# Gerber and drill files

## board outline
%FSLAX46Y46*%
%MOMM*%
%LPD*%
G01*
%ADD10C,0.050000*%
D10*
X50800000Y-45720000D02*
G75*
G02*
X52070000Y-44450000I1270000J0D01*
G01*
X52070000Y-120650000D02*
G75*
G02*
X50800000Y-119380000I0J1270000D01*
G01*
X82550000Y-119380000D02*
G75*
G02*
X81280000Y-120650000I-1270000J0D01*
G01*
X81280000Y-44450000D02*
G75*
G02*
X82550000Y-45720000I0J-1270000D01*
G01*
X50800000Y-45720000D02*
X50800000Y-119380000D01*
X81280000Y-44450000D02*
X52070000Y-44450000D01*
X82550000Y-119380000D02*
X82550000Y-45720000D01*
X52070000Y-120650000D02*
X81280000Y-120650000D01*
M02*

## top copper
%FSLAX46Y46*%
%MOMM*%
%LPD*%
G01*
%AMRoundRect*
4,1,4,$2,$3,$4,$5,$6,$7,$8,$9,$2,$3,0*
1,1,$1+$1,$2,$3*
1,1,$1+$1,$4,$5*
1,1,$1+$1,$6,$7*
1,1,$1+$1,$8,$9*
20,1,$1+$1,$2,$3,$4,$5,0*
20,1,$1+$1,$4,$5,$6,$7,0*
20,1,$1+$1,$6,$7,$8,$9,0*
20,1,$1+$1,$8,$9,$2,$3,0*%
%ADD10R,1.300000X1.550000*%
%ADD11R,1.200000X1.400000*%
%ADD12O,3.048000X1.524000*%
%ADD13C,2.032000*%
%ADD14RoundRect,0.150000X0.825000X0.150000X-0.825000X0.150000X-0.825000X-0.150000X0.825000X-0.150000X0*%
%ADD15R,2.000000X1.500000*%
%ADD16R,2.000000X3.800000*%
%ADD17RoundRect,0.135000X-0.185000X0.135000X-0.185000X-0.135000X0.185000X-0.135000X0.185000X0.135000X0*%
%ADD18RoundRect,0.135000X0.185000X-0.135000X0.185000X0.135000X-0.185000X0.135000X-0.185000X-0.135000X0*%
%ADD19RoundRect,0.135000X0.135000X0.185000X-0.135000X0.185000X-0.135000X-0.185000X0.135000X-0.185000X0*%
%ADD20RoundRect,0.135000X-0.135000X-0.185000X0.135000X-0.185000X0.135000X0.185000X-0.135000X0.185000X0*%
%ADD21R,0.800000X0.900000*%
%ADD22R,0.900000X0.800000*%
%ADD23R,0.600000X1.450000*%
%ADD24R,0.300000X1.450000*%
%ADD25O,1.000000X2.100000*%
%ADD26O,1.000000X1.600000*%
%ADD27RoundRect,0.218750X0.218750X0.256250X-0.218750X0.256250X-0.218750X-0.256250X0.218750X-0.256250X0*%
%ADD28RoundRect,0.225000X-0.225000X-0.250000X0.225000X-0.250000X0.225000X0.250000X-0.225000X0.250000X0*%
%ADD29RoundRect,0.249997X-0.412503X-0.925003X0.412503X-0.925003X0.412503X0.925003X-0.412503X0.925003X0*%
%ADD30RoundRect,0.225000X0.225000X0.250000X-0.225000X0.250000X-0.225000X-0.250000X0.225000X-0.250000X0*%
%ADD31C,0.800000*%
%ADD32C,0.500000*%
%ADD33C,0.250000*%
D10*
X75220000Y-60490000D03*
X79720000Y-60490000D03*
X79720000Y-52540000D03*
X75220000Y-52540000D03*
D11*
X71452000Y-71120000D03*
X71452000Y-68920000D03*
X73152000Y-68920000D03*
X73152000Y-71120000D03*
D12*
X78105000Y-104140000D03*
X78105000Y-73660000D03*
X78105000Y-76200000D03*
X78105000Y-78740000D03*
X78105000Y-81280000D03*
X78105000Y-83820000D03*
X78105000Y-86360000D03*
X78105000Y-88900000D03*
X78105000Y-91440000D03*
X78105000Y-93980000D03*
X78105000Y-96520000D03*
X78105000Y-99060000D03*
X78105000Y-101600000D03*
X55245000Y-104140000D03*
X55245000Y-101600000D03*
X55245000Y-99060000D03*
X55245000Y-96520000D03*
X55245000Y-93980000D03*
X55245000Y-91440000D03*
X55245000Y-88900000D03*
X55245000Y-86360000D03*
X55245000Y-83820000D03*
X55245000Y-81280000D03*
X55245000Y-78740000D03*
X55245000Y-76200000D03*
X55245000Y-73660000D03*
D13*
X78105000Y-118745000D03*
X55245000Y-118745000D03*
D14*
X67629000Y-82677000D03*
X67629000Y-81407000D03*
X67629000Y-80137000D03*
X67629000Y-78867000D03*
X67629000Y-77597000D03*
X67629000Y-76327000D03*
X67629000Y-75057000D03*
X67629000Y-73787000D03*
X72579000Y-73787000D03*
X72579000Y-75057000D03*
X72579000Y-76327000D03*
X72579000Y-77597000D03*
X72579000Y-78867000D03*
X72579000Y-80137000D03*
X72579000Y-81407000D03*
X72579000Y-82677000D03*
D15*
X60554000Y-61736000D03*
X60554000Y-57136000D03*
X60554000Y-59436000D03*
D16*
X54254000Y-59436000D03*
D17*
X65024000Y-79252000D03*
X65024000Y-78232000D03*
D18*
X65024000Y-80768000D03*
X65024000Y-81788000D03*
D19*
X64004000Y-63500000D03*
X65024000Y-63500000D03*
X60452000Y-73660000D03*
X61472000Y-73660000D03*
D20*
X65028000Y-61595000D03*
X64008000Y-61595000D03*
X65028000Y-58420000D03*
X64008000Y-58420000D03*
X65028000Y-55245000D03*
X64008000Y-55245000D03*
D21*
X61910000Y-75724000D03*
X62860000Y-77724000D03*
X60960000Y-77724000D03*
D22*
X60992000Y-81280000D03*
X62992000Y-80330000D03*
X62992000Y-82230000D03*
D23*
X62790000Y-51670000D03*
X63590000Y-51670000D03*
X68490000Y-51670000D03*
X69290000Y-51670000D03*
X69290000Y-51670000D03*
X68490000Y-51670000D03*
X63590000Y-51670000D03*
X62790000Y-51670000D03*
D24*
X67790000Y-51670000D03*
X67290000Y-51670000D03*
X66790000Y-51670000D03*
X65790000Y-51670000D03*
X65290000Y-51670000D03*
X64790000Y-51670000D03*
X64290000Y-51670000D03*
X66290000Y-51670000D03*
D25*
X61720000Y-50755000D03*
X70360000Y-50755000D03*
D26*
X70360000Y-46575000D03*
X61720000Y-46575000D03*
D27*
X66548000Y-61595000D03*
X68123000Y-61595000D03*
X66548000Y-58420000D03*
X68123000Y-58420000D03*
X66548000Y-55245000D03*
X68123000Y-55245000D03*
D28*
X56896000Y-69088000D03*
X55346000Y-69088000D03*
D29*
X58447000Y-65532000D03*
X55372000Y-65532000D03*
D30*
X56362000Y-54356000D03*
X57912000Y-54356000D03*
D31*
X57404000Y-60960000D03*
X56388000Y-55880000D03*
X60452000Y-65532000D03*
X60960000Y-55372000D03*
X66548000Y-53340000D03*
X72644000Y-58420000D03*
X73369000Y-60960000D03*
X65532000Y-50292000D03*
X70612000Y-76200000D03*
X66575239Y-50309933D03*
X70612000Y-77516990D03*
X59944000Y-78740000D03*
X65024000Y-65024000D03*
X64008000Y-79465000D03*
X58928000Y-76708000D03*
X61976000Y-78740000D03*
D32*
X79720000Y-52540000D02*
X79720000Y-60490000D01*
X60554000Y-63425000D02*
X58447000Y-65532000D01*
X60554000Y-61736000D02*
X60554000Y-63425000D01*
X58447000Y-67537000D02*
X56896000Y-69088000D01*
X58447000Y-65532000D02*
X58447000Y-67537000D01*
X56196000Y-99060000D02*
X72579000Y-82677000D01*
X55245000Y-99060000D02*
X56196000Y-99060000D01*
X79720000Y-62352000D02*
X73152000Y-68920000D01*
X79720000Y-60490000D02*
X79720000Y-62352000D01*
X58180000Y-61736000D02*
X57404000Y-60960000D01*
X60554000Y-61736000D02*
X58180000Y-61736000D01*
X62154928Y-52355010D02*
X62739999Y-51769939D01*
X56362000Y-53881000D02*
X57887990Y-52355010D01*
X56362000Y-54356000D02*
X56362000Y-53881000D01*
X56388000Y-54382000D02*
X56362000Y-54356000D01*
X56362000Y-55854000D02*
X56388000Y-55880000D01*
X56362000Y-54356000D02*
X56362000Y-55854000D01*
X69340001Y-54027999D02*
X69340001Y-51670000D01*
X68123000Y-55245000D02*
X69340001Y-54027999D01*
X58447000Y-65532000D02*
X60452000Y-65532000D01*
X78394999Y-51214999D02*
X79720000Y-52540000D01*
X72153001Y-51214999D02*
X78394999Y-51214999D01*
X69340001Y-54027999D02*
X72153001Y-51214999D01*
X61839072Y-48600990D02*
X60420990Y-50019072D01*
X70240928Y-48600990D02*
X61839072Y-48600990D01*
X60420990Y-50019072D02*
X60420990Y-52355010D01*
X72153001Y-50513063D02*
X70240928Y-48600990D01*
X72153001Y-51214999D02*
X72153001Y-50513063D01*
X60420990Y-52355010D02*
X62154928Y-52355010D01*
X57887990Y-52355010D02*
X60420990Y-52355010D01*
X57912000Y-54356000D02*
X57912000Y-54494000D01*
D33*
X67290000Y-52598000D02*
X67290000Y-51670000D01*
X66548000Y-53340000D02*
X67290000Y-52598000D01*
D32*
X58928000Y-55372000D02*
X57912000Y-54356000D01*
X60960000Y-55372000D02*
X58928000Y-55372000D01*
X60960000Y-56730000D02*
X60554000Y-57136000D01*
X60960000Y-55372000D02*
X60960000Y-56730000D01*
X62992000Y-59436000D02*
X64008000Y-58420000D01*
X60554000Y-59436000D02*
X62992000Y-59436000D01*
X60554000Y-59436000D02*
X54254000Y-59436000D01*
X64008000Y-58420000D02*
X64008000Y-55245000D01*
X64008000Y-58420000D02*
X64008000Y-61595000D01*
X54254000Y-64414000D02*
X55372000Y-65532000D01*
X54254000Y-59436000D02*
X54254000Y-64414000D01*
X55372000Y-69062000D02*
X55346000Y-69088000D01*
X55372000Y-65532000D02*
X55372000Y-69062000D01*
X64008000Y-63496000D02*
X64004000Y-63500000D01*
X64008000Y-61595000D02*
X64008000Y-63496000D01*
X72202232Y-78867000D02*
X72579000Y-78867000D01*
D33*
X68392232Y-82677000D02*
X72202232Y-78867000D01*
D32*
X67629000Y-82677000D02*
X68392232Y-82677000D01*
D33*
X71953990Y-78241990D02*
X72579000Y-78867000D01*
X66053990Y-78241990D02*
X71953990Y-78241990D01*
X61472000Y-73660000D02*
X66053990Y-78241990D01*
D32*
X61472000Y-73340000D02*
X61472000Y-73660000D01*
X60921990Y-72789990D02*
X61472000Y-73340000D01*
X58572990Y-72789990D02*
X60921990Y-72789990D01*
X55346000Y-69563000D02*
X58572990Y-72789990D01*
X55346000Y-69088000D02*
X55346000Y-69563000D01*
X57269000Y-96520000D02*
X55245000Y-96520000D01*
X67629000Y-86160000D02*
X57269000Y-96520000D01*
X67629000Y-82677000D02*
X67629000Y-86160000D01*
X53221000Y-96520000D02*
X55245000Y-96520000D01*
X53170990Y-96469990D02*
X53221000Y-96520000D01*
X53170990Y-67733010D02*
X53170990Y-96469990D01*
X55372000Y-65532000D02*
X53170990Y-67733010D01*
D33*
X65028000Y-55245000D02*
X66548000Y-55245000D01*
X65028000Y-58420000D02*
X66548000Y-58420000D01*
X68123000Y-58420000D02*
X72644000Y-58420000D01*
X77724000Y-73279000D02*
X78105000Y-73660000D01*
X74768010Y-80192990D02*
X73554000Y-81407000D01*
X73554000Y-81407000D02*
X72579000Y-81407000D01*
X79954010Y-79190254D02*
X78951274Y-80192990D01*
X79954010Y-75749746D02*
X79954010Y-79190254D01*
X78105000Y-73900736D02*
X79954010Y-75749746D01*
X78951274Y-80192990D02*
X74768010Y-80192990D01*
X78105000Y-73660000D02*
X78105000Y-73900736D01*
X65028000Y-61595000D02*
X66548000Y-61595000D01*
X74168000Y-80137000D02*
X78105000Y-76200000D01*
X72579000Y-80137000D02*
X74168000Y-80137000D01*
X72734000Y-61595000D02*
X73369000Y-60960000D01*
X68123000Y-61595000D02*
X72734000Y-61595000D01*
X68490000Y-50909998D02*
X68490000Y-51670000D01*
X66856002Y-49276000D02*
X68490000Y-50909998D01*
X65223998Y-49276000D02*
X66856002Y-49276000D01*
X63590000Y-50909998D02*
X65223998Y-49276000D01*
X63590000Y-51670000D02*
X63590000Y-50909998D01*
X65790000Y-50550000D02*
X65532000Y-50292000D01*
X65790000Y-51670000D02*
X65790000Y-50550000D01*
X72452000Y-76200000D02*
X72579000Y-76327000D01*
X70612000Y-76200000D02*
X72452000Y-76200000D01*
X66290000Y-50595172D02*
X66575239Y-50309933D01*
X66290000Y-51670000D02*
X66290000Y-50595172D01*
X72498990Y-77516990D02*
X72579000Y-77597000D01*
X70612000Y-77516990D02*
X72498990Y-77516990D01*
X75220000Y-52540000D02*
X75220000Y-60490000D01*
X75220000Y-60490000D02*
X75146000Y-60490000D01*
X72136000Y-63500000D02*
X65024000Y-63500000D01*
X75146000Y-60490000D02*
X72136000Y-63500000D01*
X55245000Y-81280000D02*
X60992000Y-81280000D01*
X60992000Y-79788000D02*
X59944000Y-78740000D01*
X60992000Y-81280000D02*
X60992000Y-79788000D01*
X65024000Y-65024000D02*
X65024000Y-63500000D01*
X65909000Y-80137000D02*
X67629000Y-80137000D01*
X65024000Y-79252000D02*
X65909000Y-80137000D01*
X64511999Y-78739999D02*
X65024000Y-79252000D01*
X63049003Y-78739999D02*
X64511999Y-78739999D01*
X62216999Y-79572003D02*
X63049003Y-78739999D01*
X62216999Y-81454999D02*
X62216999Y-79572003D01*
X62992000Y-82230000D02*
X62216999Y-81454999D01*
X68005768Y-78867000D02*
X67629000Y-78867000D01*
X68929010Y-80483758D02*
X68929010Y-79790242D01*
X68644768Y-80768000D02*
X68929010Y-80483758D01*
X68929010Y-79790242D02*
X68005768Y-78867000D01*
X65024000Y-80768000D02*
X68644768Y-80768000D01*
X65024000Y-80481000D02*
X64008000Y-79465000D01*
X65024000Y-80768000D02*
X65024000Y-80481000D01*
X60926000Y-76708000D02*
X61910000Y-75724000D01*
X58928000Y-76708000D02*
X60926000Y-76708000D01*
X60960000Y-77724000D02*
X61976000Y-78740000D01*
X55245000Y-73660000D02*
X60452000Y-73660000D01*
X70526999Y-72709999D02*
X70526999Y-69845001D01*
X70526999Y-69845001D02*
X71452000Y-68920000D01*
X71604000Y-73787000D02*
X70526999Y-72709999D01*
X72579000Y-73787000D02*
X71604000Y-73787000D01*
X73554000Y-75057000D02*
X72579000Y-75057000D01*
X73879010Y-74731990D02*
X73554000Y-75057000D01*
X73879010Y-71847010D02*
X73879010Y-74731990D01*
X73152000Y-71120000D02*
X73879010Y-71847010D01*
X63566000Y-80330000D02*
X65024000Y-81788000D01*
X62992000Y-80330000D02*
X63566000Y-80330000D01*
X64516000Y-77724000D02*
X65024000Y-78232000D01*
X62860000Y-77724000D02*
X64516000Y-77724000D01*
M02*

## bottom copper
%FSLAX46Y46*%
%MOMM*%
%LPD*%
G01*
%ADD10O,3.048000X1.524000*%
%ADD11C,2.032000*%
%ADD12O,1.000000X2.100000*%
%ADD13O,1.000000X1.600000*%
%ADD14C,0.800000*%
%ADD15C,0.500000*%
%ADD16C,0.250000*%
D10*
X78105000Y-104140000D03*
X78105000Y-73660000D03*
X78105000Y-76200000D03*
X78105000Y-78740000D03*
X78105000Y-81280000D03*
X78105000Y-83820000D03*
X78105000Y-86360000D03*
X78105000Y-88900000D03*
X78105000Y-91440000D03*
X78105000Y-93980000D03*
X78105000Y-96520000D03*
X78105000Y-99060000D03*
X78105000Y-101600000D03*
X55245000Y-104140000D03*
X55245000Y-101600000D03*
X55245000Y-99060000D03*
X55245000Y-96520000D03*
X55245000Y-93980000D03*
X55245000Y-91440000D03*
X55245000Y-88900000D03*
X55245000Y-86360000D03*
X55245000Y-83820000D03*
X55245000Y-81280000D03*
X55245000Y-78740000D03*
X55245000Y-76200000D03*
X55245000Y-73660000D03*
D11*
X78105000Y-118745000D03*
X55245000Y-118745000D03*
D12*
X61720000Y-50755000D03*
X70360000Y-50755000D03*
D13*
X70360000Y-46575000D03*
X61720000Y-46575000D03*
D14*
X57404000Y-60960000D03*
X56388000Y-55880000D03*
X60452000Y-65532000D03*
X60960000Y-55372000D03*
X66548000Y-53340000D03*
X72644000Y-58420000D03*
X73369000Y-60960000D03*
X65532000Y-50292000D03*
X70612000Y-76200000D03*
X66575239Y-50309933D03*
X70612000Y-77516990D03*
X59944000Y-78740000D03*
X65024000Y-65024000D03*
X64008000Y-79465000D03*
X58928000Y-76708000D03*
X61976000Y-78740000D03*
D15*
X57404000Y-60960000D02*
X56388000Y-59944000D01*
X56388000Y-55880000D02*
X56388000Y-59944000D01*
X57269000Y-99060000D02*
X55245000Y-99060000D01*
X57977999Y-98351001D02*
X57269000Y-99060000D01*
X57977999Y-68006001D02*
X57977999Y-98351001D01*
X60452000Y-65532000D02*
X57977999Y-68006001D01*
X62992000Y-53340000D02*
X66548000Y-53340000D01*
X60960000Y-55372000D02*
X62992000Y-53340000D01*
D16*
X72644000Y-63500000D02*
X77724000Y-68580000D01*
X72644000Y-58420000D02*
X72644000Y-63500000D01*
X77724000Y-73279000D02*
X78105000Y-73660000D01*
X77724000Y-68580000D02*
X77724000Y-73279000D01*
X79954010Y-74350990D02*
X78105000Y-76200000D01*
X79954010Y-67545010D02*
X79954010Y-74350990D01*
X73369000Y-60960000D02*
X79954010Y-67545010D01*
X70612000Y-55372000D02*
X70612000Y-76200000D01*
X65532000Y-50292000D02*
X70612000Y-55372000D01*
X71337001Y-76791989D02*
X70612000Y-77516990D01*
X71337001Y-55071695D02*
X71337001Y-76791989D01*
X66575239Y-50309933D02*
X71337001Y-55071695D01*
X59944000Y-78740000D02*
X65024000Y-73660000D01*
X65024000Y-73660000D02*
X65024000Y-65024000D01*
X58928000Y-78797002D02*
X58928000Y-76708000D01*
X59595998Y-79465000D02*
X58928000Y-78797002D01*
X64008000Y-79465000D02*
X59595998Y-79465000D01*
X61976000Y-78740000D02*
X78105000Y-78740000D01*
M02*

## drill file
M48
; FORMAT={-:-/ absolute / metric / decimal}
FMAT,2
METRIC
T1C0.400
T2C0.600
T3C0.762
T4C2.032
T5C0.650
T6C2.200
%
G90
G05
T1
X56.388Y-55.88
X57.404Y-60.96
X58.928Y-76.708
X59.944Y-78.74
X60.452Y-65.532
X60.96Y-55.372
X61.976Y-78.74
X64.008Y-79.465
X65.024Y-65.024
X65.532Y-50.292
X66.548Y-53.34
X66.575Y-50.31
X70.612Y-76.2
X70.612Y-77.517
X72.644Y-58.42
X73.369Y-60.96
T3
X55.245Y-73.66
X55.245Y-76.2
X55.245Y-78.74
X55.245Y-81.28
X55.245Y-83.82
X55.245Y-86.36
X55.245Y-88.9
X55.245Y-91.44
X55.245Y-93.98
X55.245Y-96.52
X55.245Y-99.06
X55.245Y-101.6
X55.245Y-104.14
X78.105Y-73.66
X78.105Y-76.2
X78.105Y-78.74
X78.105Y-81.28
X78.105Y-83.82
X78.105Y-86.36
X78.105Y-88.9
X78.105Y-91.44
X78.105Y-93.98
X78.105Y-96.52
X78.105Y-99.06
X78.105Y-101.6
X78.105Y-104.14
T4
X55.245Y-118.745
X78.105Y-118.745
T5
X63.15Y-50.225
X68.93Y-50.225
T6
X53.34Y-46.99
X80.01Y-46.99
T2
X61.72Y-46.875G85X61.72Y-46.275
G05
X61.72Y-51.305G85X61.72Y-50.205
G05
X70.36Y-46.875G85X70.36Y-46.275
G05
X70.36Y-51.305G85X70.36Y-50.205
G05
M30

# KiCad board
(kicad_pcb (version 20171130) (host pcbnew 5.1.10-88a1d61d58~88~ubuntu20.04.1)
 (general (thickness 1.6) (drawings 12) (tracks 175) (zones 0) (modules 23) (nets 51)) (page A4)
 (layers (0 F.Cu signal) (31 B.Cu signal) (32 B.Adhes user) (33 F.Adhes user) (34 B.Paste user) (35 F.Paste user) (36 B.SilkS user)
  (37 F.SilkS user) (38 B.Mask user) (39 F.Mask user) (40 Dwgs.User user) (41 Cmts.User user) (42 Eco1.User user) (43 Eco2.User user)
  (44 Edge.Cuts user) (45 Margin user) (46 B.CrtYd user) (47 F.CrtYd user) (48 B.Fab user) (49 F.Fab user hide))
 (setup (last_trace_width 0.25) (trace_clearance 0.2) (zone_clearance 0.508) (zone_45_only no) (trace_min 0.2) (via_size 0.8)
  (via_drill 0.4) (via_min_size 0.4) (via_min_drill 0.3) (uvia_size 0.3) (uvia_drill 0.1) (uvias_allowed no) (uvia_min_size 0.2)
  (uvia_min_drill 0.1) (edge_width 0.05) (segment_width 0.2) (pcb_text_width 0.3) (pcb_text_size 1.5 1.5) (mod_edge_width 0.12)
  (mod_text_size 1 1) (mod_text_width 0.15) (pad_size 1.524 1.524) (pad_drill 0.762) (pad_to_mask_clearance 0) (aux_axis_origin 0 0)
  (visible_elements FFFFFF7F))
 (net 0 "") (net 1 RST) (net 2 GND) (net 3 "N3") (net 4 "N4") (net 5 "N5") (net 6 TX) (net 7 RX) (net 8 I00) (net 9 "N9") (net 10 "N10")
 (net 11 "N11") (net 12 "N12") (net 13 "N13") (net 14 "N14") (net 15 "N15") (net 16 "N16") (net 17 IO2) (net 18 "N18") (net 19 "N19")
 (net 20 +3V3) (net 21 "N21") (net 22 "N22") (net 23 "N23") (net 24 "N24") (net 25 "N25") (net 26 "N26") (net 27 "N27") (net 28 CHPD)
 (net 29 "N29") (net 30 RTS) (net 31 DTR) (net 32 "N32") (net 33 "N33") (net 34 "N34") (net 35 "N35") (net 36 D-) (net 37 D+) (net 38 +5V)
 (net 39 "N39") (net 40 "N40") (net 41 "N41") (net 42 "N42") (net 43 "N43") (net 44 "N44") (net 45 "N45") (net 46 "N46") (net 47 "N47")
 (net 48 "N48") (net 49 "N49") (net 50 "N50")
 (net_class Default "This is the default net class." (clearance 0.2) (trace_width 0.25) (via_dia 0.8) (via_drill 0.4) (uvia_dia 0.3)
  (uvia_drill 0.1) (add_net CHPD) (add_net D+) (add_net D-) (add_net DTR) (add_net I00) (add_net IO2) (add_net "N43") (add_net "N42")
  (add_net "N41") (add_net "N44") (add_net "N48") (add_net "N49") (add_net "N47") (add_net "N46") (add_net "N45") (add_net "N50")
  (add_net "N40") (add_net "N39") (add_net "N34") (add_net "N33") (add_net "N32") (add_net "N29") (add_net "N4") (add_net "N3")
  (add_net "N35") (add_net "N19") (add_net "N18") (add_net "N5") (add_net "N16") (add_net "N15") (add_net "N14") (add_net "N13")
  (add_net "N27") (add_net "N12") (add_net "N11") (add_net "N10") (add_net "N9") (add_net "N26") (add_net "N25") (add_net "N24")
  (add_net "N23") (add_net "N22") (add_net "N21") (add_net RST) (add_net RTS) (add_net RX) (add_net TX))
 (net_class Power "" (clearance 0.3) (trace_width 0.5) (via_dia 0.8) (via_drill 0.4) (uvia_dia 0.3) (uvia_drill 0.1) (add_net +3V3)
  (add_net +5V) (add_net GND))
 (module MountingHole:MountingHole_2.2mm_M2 (layer F.Cu) (at 53.34 46.99)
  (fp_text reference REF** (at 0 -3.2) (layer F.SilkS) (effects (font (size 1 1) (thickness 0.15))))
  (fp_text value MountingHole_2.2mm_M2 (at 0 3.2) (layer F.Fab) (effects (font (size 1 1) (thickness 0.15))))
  (pad 1 np_thru_hole circle (at 0 0) (size 2.2 2.2) (drill 2.2) (layers *.Cu *.Mask)))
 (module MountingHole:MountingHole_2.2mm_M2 (layer F.Cu) (at 80.01 46.99)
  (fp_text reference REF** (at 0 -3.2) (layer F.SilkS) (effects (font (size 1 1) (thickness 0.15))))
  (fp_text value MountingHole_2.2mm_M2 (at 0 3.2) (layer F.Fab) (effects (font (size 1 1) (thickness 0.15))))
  (pad 1 np_thru_hole circle (at 0 0) (size 2.2 2.2) (drill 2.2) (layers *.Cu *.Mask)))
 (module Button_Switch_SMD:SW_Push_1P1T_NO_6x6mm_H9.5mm (layer F.Cu) (at 77.47 56.515 270)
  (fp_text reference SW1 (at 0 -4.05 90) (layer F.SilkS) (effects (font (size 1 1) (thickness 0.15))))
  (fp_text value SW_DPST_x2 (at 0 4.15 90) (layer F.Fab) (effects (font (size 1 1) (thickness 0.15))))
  (pad 2 smd rect (at 3.975 2.25 270) (size 1.55 1.3) (layers F.Cu F.Paste F.Mask) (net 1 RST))
  (pad 1 smd rect (at 3.975 -2.25 270) (size 1.55 1.3) (layers F.Cu F.Paste F.Mask) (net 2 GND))
  (pad 1 smd rect (at -3.975 -2.25 270) (size 1.55 1.3) (layers F.Cu F.Paste F.Mask) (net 2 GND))
  (pad 2 smd rect (at -3.975 2.25 270) (size 1.55 1.3) (layers F.Cu F.Paste F.Mask) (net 1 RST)))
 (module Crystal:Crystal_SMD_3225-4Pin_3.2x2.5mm (layer F.Cu) (at 72.302 70.02 90)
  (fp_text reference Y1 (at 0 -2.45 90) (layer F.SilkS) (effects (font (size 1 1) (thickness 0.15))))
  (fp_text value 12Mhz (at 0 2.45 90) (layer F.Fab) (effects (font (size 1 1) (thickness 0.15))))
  (pad 4 smd rect (at -1.1 -0.85 90) (size 1.4 1.2) (layers F.Cu F.Paste F.Mask))
  (pad 3 smd rect (at 1.1 -0.85 90) (size 1.4 1.2) (layers F.Cu F.Paste F.Mask) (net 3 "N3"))
  (pad 2 smd rect (at 1.1 0.85 90) (size 1.4 1.2) (layers F.Cu F.Paste F.Mask) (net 2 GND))
  (pad 1 smd rect (at -1.1 0.85 90) (size 1.4 1.2) (layers F.Cu F.Paste F.Mask) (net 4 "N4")))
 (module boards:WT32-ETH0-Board (layer F.Cu) (at 66.675 92.71)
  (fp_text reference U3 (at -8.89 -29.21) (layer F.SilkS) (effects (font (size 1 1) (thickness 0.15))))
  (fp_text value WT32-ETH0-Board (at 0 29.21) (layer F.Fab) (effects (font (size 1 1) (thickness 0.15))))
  (pad 14 thru_hole oval (at 11.43 11.43) (size 3.048 1.524) (drill 0.762) (layers *.Cu *.Mask) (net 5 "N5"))
  (pad 26 thru_hole oval (at 11.43 -19.05) (size 3.048 1.524) (drill 0.762) (layers *.Cu *.Mask) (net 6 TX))
  (pad 25 thru_hole oval (at 11.43 -16.51) (size 3.048 1.524) (drill 0.762) (layers *.Cu *.Mask) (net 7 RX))
  (pad 24 thru_hole oval (at 11.43 -13.97) (size 3.048 1.524) (drill 0.762) (layers *.Cu *.Mask) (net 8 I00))
  (pad 23 thru_hole oval (at 11.43 -11.43) (size 3.048 1.524) (drill 0.762) (layers *.Cu *.Mask) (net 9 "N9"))
  (pad 22 thru_hole oval (at 11.43 -8.89) (size 3.048 1.524) (drill 0.762) (layers *.Cu *.Mask) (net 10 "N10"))
  (pad 21 thru_hole oval (at 11.43 -6.35) (size 3.048 1.524) (drill 0.762) (layers *.Cu *.Mask) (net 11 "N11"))
  (pad 20 thru_hole oval (at 11.43 -3.81) (size 3.048 1.524) (drill 0.762) (layers *.Cu *.Mask) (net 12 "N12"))
  (pad 19 thru_hole oval (at 11.43 -1.27) (size 3.048 1.524) (drill 0.762) (layers *.Cu *.Mask) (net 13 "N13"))
  (pad 18 thru_hole oval (at 11.43 1.27) (size 3.048 1.524) (drill 0.762) (layers *.Cu *.Mask) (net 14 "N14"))
  (pad 17 thru_hole oval (at 11.43 3.81) (size 3.048 1.524) (drill 0.762) (layers *.Cu *.Mask) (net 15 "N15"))
  (pad 16 thru_hole oval (at 11.43 6.35) (size 3.048 1.524) (drill 0.762) (layers *.Cu *.Mask) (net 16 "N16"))
  (pad 15 thru_hole oval (at 11.43 8.89) (size 3.048 1.524) (drill 0.762) (layers *.Cu *.Mask) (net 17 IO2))
  (pad 13 thru_hole oval (at -11.43 11.43) (size 3.048 1.524) (drill 0.762) (layers *.Cu *.Mask) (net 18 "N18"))
  (pad 12 thru_hole oval (at -11.43 8.89) (size 3.048 1.524) (drill 0.762) (layers *.Cu *.Mask) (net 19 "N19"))
  (pad 11 thru_hole oval (at -11.43 6.35) (size 3.048 1.524) (drill 0.762) (layers *.Cu *.Mask) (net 2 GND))
  (pad 10 thru_hole oval (at -11.43 3.81) (size 3.048 1.524) (drill 0.762) (layers *.Cu *.Mask) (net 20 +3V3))
  (pad 9 thru_hole oval (at -11.43 1.27) (size 3.048 1.524) (drill 0.762) (layers *.Cu *.Mask) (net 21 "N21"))
  (pad 8 thru_hole oval (at -11.43 -1.27) (size 3.048 1.524) (drill 0.762) (layers *.Cu *.Mask) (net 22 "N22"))
  (pad 7 thru_hole oval (at -11.43 -3.81) (size 3.048 1.524) (drill 0.762) (layers *.Cu *.Mask) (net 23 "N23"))
  (pad 6 thru_hole oval (at -11.43 -6.35) (size 3.048 1.524) (drill 0.762) (layers *.Cu *.Mask) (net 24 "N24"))
  (pad 5 thru_hole oval (at -11.43 -8.89) (size 3.048 1.524) (drill 0.762) (layers *.Cu *.Mask) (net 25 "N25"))
  (pad 4 thru_hole oval (at -11.43 -11.43) (size 3.048 1.524) (drill 0.762) (layers *.Cu *.Mask) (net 1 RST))
  (pad 3 thru_hole oval (at -11.43 -13.97) (size 3.048 1.524) (drill 0.762) (layers *.Cu *.Mask) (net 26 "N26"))
  (pad 2 thru_hole oval (at -11.43 -16.51) (size 3.048 1.524) (drill 0.762) (layers *.Cu *.Mask) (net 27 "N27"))
  (pad 1 thru_hole oval (at -11.43 -19.05) (size 3.048 1.524) (drill 0.762) (layers *.Cu *.Mask) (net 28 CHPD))
  (pad "" thru_hole circle (at 11.43 26.035) (size 2.032 2.032) (drill 2.032) (layers *.Mask F.Cu))
  (pad "" thru_hole circle (at -11.43 26.035) (size 2.032 2.032) (drill 2.032) (layers *.Mask F.Cu)))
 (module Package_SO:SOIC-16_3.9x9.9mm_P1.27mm (layer F.Cu) (at 70.104 78.232 180)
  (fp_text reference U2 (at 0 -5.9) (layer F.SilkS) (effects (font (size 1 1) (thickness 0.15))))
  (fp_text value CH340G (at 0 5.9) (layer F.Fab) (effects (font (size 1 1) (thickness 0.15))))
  (pad 16 smd roundrect (at 2.475 -4.445 180) (size 1.95 0.6) (layers F.Cu F.Paste F.Mask) (roundrect_rratio 0.25) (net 20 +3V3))
  (pad 15 smd roundrect (at 2.475 -3.175 180) (size 1.95 0.6) (layers F.Cu F.Paste F.Mask) (roundrect_rratio 0.25) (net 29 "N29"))
  (pad 14 smd roundrect (at 2.475 -1.905 180) (size 1.95 0.6) (layers F.Cu F.Paste F.Mask) (roundrect_rratio 0.25) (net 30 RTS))
  (pad 13 smd roundrect (at 2.475 -0.635 180) (size 1.95 0.6) (layers F.Cu F.Paste F.Mask) (roundrect_rratio 0.25) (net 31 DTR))
  (pad 12 smd roundrect (at 2.475 0.635 180) (size 1.95 0.6) (layers F.Cu F.Paste F.Mask) (roundrect_rratio 0.25) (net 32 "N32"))
  (pad 11 smd roundrect (at 2.475 1.905 180) (size 1.95 0.6) (layers F.Cu F.Paste F.Mask) (roundrect_rratio 0.25) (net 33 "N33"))
  (pad 10 smd roundrect (at 2.475 3.175 180) (size 1.95 0.6) (layers F.Cu F.Paste F.Mask) (roundrect_rratio 0.25) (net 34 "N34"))
  (pad 9 smd roundrect (at 2.475 4.445 180) (size 1.95 0.6) (layers F.Cu F.Paste F.Mask) (roundrect_rratio 0.25) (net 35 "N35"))
  (pad 8 smd roundrect (at -2.475 4.445 180) (size 1.95 0.6) (layers F.Cu F.Paste F.Mask) (roundrect_rratio 0.25) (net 3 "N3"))
  (pad 7 smd roundrect (at -2.475 3.175 180) (size 1.95 0.6) (layers F.Cu F.Paste F.Mask) (roundrect_rratio 0.25) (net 4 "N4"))
  (pad 6 smd roundrect (at -2.475 1.905 180) (size 1.95 0.6) (layers F.Cu F.Paste F.Mask) (roundrect_rratio 0.25) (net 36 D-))
  (pad 5 smd roundrect (at -2.475 0.635 180) (size 1.95 0.6) (layers F.Cu F.Paste F.Mask) (roundrect_rratio 0.25) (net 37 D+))
  (pad 4 smd roundrect (at -2.475 -0.635 180) (size 1.95 0.6) (layers F.Cu F.Paste F.Mask) (roundrect_rratio 0.25) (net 20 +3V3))
  (pad 3 smd roundrect (at -2.475 -1.905 180) (size 1.95 0.6) (layers F.Cu F.Paste F.Mask) (roundrect_rratio 0.25) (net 7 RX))
  (pad 2 smd roundrect (at -2.475 -3.175 180) (size 1.95 0.6) (layers F.Cu F.Paste F.Mask) (roundrect_rratio 0.25) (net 6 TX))
  (pad 1 smd roundrect (at -2.475 -4.445 180) (size 1.95 0.6) (layers F.Cu F.Paste F.Mask) (roundrect_rratio 0.25) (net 2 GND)))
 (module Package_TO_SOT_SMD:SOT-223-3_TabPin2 (layer F.Cu) (at 57.404 59.436 180)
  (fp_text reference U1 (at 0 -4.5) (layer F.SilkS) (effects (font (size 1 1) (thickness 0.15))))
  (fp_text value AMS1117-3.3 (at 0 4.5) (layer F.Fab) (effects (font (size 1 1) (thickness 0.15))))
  (pad 1 smd rect (at -3.15 -2.3 180) (size 2 1.5) (layers F.Cu F.Paste F.Mask) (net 2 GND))
  (pad 3 smd rect (at -3.15 2.3 180) (size 2 1.5) (layers F.Cu F.Paste F.Mask) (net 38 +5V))
  (pad 2 smd rect (at -3.15 0 180) (size 2 1.5) (layers F.Cu F.Paste F.Mask) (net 20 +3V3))
  (pad 2 smd rect (at 3.15 0 180) (size 2 3.8) (layers F.Cu F.Paste F.Mask) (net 20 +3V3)))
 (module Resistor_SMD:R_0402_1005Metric (layer F.Cu) (at 65.024 78.742 270)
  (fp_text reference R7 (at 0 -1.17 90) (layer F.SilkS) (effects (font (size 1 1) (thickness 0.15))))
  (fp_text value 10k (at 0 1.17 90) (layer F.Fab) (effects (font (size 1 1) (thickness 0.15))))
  (pad 2 smd roundrect (at 0.51 0 270) (size 0.54 0.64) (layers F.Cu F.Paste F.Mask) (roundrect_rratio 0.25) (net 30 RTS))
  (pad 1 smd roundrect (at -0.51 0 270) (size 0.54 0.64) (layers F.Cu F.Paste F.Mask) (roundrect_rratio 0.25) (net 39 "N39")))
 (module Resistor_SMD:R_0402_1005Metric (layer F.Cu) (at 65.024 81.278 90)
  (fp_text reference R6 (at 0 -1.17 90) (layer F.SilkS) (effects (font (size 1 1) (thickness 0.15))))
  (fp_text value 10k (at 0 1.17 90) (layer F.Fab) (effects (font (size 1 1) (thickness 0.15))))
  (pad 2 smd roundrect (at 0.51 0 90) (size 0.54 0.64) (layers F.Cu F.Paste F.Mask) (roundrect_rratio 0.25) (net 31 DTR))
  (pad 1 smd roundrect (at -0.51 0 90) (size 0.54 0.64) (layers F.Cu F.Paste F.Mask) (roundrect_rratio 0.25) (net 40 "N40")))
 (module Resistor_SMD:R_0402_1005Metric (layer F.Cu) (at 64.514 63.5 180)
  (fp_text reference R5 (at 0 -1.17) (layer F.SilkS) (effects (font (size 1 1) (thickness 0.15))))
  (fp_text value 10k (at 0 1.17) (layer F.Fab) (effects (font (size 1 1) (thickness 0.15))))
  (pad 2 smd roundrect (at 0.51 0 180) (size 0.54 0.64) (layers F.Cu F.Paste F.Mask) (roundrect_rratio 0.25) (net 20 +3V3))
  (pad 1 smd roundrect (at -0.51 0 180) (size 0.54 0.64) (layers F.Cu F.Paste F.Mask) (roundrect_rratio 0.25) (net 1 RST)))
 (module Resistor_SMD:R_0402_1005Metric (layer F.Cu) (at 60.962 73.66 180)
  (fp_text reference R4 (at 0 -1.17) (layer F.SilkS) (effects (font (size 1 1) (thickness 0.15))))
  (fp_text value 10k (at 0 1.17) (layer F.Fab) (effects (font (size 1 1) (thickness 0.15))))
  (pad 2 smd roundrect (at 0.51 0 180) (size 0.54 0.64) (layers F.Cu F.Paste F.Mask) (roundrect_rratio 0.25) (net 28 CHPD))
  (pad 1 smd roundrect (at -0.51 0 180) (size 0.54 0.64) (layers F.Cu F.Paste F.Mask) (roundrect_rratio 0.25) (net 20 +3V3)))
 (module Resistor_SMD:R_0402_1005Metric (layer F.Cu) (at 64.518 61.595)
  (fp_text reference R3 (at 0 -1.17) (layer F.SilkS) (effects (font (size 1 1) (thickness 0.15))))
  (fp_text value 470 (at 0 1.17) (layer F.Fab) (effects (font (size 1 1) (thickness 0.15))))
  (pad 2 smd roundrect (at 0.51 0) (size 0.54 0.64) (layers F.Cu F.Paste F.Mask) (roundrect_rratio 0.25) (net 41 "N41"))
  (pad 1 smd roundrect (at -0.51 0) (size 0.54 0.64) (layers F.Cu F.Paste F.Mask) (roundrect_rratio 0.25) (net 20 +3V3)))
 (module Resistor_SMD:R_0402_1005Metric (layer F.Cu) (at 64.518 58.42)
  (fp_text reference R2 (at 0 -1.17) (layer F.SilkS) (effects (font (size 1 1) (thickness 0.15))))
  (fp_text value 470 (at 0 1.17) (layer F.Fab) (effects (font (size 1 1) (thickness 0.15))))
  (pad 2 smd roundrect (at 0.51 0) (size 0.54 0.64) (layers F.Cu F.Paste F.Mask) (roundrect_rratio 0.25) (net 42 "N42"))
  (pad 1 smd roundrect (at -0.51 0) (size 0.54 0.64) (layers F.Cu F.Paste F.Mask) (roundrect_rratio 0.25) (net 20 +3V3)))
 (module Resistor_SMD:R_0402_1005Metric (layer F.Cu) (at 64.518 55.245)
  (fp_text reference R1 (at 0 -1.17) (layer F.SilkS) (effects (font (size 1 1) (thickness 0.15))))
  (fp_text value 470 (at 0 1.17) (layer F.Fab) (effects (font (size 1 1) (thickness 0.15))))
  (pad 2 smd roundrect (at 0.51 0) (size 0.54 0.64) (layers F.Cu F.Paste F.Mask) (roundrect_rratio 0.25) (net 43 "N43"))
  (pad 1 smd roundrect (at -0.51 0) (size 0.54 0.64) (layers F.Cu F.Paste F.Mask) (roundrect_rratio 0.25) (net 20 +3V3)))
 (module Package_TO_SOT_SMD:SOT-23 (layer F.Cu) (at 61.91 76.724 90)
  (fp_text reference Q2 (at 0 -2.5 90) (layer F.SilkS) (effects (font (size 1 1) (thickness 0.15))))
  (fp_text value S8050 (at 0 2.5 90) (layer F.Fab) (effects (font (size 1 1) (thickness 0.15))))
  (pad 3 smd rect (at 1 0 90) (size 0.9 0.8) (layers F.Cu F.Paste F.Mask) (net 31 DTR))
  (pad 2 smd rect (at -1 0.95 90) (size 0.9 0.8) (layers F.Cu F.Paste F.Mask) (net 39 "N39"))
  (pad 1 smd rect (at -1 -0.95 90) (size 0.9 0.8) (layers F.Cu F.Paste F.Mask) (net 8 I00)))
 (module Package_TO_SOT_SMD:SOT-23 (layer F.Cu) (at 61.992 81.28 180)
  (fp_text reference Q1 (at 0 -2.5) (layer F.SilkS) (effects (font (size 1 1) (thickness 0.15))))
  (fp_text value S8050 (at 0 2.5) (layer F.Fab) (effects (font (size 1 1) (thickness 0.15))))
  (pad 3 smd rect (at 1 0 180) (size 0.9 0.8) (layers F.Cu F.Paste F.Mask) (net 1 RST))
  (pad 2 smd rect (at -1 0.95 180) (size 0.9 0.8) (layers F.Cu F.Paste F.Mask) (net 40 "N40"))
  (pad 1 smd rect (at -1 -0.95 180) (size 0.9 0.8) (layers F.Cu F.Paste F.Mask) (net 30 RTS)))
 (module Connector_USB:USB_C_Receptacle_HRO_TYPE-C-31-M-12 (layer F.Cu) (at 66.04 47.625 180)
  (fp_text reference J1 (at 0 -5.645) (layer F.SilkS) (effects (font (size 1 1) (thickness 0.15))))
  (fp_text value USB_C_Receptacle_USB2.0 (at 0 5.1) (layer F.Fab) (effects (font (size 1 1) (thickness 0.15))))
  (pad B1 smd rect (at 3.25 -4.045 180) (size 0.6 1.45) (layers F.Cu F.Paste F.Mask) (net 2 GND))
  (pad A9 smd rect (at 2.45 -4.045 180) (size 0.6 1.45) (layers F.Cu F.Paste F.Mask) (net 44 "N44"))
  (pad B9 smd rect (at -2.45 -4.045 180) (size 0.6 1.45) (layers F.Cu F.Paste F.Mask) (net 44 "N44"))
  (pad B12 smd rect (at -3.25 -4.045 180) (size 0.6 1.45) (layers F.Cu F.Paste F.Mask) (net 2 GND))
  (pad A1 smd rect (at -3.25 -4.045 180) (size 0.6 1.45) (layers F.Cu F.Paste F.Mask) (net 2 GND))
  (pad A4 smd rect (at -2.45 -4.045 180) (size 0.6 1.45) (layers F.Cu F.Paste F.Mask) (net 44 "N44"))
  (pad B4 smd rect (at 2.45 -4.045 180) (size 0.6 1.45) (layers F.Cu F.Paste F.Mask) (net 44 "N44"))
  (pad A12 smd rect (at 3.25 -4.045 180) (size 0.6 1.45) (layers F.Cu F.Paste F.Mask) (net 2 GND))
  (pad B8 smd rect (at -1.75 -4.045 180) (size 0.3 1.45) (layers F.Cu F.Paste F.Mask) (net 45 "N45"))
  (pad A5 smd rect (at -1.25 -4.045 180) (size 0.3 1.45) (layers F.Cu F.Paste F.Mask) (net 38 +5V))
  (pad B7 smd rect (at -0.75 -4.045 180) (size 0.3 1.45) (layers F.Cu F.Paste F.Mask) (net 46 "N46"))
  (pad A7 smd rect (at 0.25 -4.045 180) (size 0.3 1.45) (layers F.Cu F.Paste F.Mask) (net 36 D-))
  (pad B6 smd rect (at 0.75 -4.045 180) (size 0.3 1.45) (layers F.Cu F.Paste F.Mask) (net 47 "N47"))
  (pad A8 smd rect (at 1.25 -4.045 180) (size 0.3 1.45) (layers F.Cu F.Paste F.Mask) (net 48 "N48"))
  (pad B5 smd rect (at 1.75 -4.045 180) (size 0.3 1.45) (layers F.Cu F.Paste F.Mask) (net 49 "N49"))
  (pad A6 smd rect (at -0.25 -4.045 180) (size 0.3 1.45) (layers F.Cu F.Paste F.Mask) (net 37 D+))
  (pad S1 thru_hole oval (at 4.32 -3.13 180) (size 1 2.1) (drill oval 0.6 1.7) (layers *.Cu *.Mask) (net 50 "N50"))
  (pad S1 thru_hole oval (at -4.32 -3.13 180) (size 1 2.1) (drill oval 0.6 1.7) (layers *.Cu *.Mask) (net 50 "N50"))
  (pad "" np_thru_hole circle (at -2.89 -2.6 180) (size 0.65 0.65) (drill 0.65) (layers *.Cu *.Mask))
  (pad S1 thru_hole oval (at -4.32 1.05 180) (size 1 1.6) (drill oval 0.6 1.2) (layers *.Cu *.Mask) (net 50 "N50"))
  (pad "" np_thru_hole circle (at 2.89 -2.6 180) (size 0.65 0.65) (drill 0.65) (layers *.Cu *.Mask))
  (pad S1 thru_hole oval (at 4.32 1.05 180) (size 1 1.6) (drill oval 0.6 1.2) (layers *.Cu *.Mask) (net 50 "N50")))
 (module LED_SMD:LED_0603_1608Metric (layer F.Cu) (at 67.3355 61.595 180)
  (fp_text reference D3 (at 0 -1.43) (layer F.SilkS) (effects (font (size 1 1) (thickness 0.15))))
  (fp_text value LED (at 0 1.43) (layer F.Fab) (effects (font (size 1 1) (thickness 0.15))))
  (pad 2 smd roundrect (at 0.7875 0 180) (size 0.875 0.95) (layers F.Cu F.Paste F.Mask) (roundrect_rratio 0.25) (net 41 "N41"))
  (pad 1 smd roundrect (at -0.7875 0 180) (size 0.875 0.95) (layers F.Cu F.Paste F.Mask) (roundrect_rratio 0.25) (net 7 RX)))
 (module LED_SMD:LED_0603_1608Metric (layer F.Cu) (at 67.3355 58.42 180)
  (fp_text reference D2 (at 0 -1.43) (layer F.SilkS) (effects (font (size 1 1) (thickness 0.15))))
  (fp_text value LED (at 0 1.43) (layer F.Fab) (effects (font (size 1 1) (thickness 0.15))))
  (pad 2 smd roundrect (at 0.7875 0 180) (size 0.875 0.95) (layers F.Cu F.Paste F.Mask) (roundrect_rratio 0.25) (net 42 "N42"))
  (pad 1 smd roundrect (at -0.7875 0 180) (size 0.875 0.95) (layers F.Cu F.Paste F.Mask) (roundrect_rratio 0.25) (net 6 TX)))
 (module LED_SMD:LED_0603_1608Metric (layer F.Cu) (at 67.3355 55.245 180)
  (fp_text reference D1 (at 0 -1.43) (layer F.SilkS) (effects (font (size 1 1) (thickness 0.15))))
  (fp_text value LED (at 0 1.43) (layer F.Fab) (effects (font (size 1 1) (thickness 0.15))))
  (pad 2 smd roundrect (at 0.7875 0 180) (size 0.875 0.95) (layers F.Cu F.Paste F.Mask) (roundrect_rratio 0.25) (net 43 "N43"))
  (pad 1 smd roundrect (at -0.7875 0 180) (size 0.875 0.95) (layers F.Cu F.Paste F.Mask) (roundrect_rratio 0.25) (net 2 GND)))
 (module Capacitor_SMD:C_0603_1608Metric (layer F.Cu) (at 56.121 69.088)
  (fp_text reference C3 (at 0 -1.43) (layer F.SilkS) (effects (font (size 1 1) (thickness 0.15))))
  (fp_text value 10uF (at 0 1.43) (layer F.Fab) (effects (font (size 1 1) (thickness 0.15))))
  (pad 2 smd roundrect (at 0.775 0) (size 0.9 0.95) (layers F.Cu F.Paste F.Mask) (roundrect_rratio 0.25) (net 2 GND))
  (pad 1 smd roundrect (at -0.775 0) (size 0.9 0.95) (layers F.Cu F.Paste F.Mask) (roundrect_rratio 0.25) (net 20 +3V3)))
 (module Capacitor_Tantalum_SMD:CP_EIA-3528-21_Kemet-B (layer F.Cu) (at 56.9095 65.532)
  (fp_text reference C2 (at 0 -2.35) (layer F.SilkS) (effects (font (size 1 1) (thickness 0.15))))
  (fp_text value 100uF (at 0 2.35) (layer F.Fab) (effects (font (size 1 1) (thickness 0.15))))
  (pad 2 smd roundrect (at 1.5375 0) (size 1.325 2.35) (layers F.Cu F.Paste F.Mask) (roundrect_rratio 0.1886769811320755) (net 2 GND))
  (pad 1 smd roundrect (at -1.5375 0) (size 1.325 2.35) (layers F.Cu F.Paste F.Mask) (roundrect_rratio 0.1886769811320755) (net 20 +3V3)))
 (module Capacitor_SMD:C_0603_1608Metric (layer F.Cu) (at 57.137 54.356 180)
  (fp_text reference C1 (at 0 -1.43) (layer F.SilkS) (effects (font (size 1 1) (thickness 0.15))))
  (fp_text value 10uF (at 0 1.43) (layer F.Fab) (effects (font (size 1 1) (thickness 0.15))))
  (pad 2 smd roundrect (at 0.775 0 180) (size 0.9 0.95) (layers F.Cu F.Paste F.Mask) (roundrect_rratio 0.25) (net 2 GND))
  (pad 1 smd roundrect (at -0.775 0 180) (size 0.9 0.95) (layers F.Cu F.Paste F.Mask) (roundrect_rratio 0.25) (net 38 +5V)))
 (gr_arc (start 52.07 45.72) (end 52.07 44.45) (angle -90) (layer Edge.Cuts) (width 0.05))
 (gr_arc (start 52.07 119.38) (end 50.8 119.38) (angle -90) (layer Edge.Cuts) (width 0.05))
 (gr_arc (start 81.28 119.38) (end 81.28 120.65) (angle -90) (layer Edge.Cuts) (width 0.05))
 (gr_arc (start 81.28 45.72) (end 82.55 45.72) (angle -90) (layer Edge.Cuts) (width 0.05))
 (gr_line (start 50.8 45.72) (end 50.8 119.38) (layer Edge.Cuts) (width 0.05))
 (gr_line (start 81.28 44.45) (end 52.07 44.45) (layer Edge.Cuts) (width 0.05))
 (gr_line (start 82.55 119.38) (end 82.55 45.72) (layer Edge.Cuts) (width 0.05))
 (gr_line (start 52.07 120.65) (end 81.28 120.65) (layer Edge.Cuts) (width 0.05))
 (segment (start 79.72 52.54) (end 79.72 60.49) (width 0.5) (layer F.Cu) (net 2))
 (segment (start 60.554 63.425) (end 58.447 65.532) (width 0.5) (layer F.Cu) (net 2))
 (segment (start 60.554 61.736) (end 60.554 63.425) (width 0.5) (layer F.Cu) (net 2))
 (segment (start 58.447 67.537) (end 56.896 69.088) (width 0.5) (layer F.Cu) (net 2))
 (segment (start 58.447 65.532) (end 58.447 67.537) (width 0.5) (layer F.Cu) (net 2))
 (segment (start 56.196 99.06) (end 72.579 82.677) (width 0.5) (layer F.Cu) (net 2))
 (segment (start 55.245 99.06) (end 56.196 99.06) (width 0.5) (layer F.Cu) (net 2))
 (segment (start 79.72 62.352) (end 73.152 68.92) (width 0.5) (layer F.Cu) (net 2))
 (segment (start 79.72 60.49) (end 79.72 62.352) (width 0.5) (layer F.Cu) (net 2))
 (via (at 57.404 60.96) (size 0.8) (drill 0.4) (layers F.Cu B.Cu) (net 2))
 (segment (start 58.18 61.736) (end 57.404 60.96) (width 0.5) (layer F.Cu) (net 2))
 (segment (start 60.554 61.736) (end 58.18 61.736) (width 0.5) (layer F.Cu) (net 2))
 (via (at 56.388 55.88) (size 0.8) (drill 0.4) (layers F.Cu B.Cu) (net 2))
 (segment (start 57.404 60.96) (end 56.388 59.944) (width 0.5) (layer B.Cu) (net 2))
 (segment (start 62.154928 52.35501) (end 62.739999 51.769939) (width 0.5) (layer F.Cu) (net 2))
 (segment (start 56.362 53.881) (end 57.88799 52.35501) (width 0.5) (layer F.Cu) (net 2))
 (segment (start 56.362 54.356) (end 56.362 53.881) (width 0.5) (layer F.Cu) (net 2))
 (segment (start 56.388 54.382) (end 56.362 54.356) (width 0.5) (layer F.Cu) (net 2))
 (segment (start 56.362 55.854) (end 56.388 55.88) (width 0.5) (layer F.Cu) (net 2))
 (segment (start 56.362 54.356) (end 56.362 55.854) (width 0.5) (layer F.Cu) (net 2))
 (segment (start 56.388 55.88) (end 56.388 59.944) (width 0.5) (layer B.Cu) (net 2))
 (segment (start 69.340001 54.027999) (end 69.340001 51.67) (width 0.5) (layer F.Cu) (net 2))
 (segment (start 68.123 55.245) (end 69.340001 54.027999) (width 0.5) (layer F.Cu) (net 2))
 (via (at 60.452 65.532) (size 0.8) (drill 0.4) (layers F.Cu B.Cu) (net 2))
 (segment (start 58.447 65.532) (end 60.452 65.532) (width 0.5) (layer F.Cu) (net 2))
 (segment (start 57.269 99.06) (end 55.245 99.06) (width 0.5) (layer B.Cu) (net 2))
 (segment (start 57.977999 98.351001) (end 57.269 99.06) (width 0.5) (layer B.Cu) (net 2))
 (segment (start 57.977999 68.006001) (end 57.977999 98.351001) (width 0.5) (layer B.Cu) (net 2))
 (segment (start 60.452 65.532) (end 57.977999 68.006001) (width 0.5) (layer B.Cu) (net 2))
 (segment (start 78.394999 51.214999) (end 79.72 52.54) (width 0.5) (layer F.Cu) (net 2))
 (segment (start 72.153001 51.214999) (end 78.394999 51.214999) (width 0.5) (layer F.Cu) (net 2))
 (segment (start 69.340001 54.027999) (end 72.153001 51.214999) (width 0.5) (layer F.Cu) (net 2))
 (segment (start 61.839072 48.60099) (end 60.42099 50.019072) (width 0.5) (layer F.Cu) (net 2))
 (segment (start 70.240928 48.60099) (end 61.839072 48.60099) (width 0.5) (layer F.Cu) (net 2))
 (segment (start 60.42099 50.019072) (end 60.42099 52.35501) (width 0.5) (layer F.Cu) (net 2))
 (segment (start 72.153001 50.513063) (end 70.240928 48.60099) (width 0.5) (layer F.Cu) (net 2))
 (segment (start 72.153001 51.214999) (end 72.153001 50.513063) (width 0.5) (layer F.Cu) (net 2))
 (segment (start 60.42099 52.35501) (end 62.154928 52.35501) (width 0.5) (layer F.Cu) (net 2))
 (segment (start 57.88799 52.35501) (end 60.42099 52.35501) (width 0.5) (layer F.Cu) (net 2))
 (segment (start 57.912 54.356) (end 57.912 54.494) (width 0.5) (layer F.Cu) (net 38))
 (via (at 60.96 55.372) (size 0.8) (drill 0.4) (layers F.Cu B.Cu) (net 38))
 (via (at 66.548 53.34) (size 0.8) (drill 0.4) (layers F.Cu B.Cu) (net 38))
 (segment (start 62.992 53.34) (end 66.548 53.34) (width 0.5) (layer B.Cu) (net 38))
 (segment (start 60.96 55.372) (end 62.992 53.34) (width 0.5) (layer B.Cu) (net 38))
 (segment (start 67.29 52.598) (end 67.29 51.67) (width 0.25) (layer F.Cu) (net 38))
 (segment (start 66.548 53.34) (end 67.29 52.598) (width 0.25) (layer F.Cu) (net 38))
 (segment (start 58.928 55.372) (end 57.912 54.356) (width 0.5) (layer F.Cu) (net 38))
 (segment (start 60.96 55.372) (end 58.928 55.372) (width 0.5) (layer F.Cu) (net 38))
 (segment (start 60.96 56.73) (end 60.554 57.136) (width 0.5) (layer F.Cu) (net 38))
 (segment (start 60.96 55.372) (end 60.96 56.73) (width 0.5) (layer F.Cu) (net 38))
 (segment (start 62.992 59.436) (end 64.008 58.42) (width 0.5) (layer F.Cu) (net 20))
 (segment (start 60.554 59.436) (end 62.992 59.436) (width 0.5) (layer F.Cu) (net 20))
 (segment (start 60.554 59.436) (end 54.254 59.436) (width 0.5) (layer F.Cu) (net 20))
 (segment (start 64.008 58.42) (end 64.008 55.245) (width 0.5) (layer F.Cu) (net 20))
 (segment (start 64.008 58.42) (end 64.008 61.595) (width 0.5) (layer F.Cu) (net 20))
 (segment (start 54.254 64.414) (end 55.372 65.532) (width 0.5) (layer F.Cu) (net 20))
 (segment (start 54.254 59.436) (end 54.254 64.414) (width 0.5) (layer F.Cu) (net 20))
 (segment (start 55.372 69.062) (end 55.346 69.088) (width 0.5) (layer F.Cu) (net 20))
 (segment (start 55.372 65.532) (end 55.372 69.062) (width 0.5) (layer F.Cu) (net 20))
 (segment (start 64.008 63.496) (end 64.004 63.5) (width 0.5) (layer F.Cu) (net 20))
 (segment (start 64.008 61.595) (end 64.008 63.496) (width 0.5) (layer F.Cu) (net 20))
 (segment (start 72.202232 78.867) (end 72.579 78.867) (width 0.5) (layer F.Cu) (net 20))
 (segment (start 68.392232 82.677) (end 72.202232 78.867) (width 0.25) (layer F.Cu) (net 20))
 (segment (start 67.629 82.677) (end 68.392232 82.677) (width 0.5) (layer F.Cu) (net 20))
 (segment (start 71.95399 78.24199) (end 72.579 78.867) (width 0.25) (layer F.Cu) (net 20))
 (segment (start 66.05399 78.24199) (end 71.95399 78.24199) (width 0.25) (layer F.Cu) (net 20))
 (segment (start 61.472 73.66) (end 66.05399 78.24199) (width 0.25) (layer F.Cu) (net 20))
 (segment (start 61.472 73.34) (end 61.472 73.66) (width 0.5) (layer F.Cu) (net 20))
 (segment (start 60.92199 72.78999) (end 61.472 73.34) (width 0.5) (layer F.Cu) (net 20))
 (segment (start 58.57299 72.78999) (end 60.92199 72.78999) (width 0.5) (layer F.Cu) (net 20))
 (segment (start 55.346 69.563) (end 58.57299 72.78999) (width 0.5) (layer F.Cu) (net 20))
 (segment (start 55.346 69.088) (end 55.346 69.563) (width 0.5) (layer F.Cu) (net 20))
 (segment (start 57.269 96.52) (end 55.245 96.52) (width 0.5) (layer F.Cu) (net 20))
 (segment (start 67.629 86.16) (end 57.269 96.52) (width 0.5) (layer F.Cu) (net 20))
 (segment (start 67.629 82.677) (end 67.629 86.16) (width 0.5) (layer F.Cu) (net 20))
 (segment (start 53.221 96.52) (end 55.245 96.52) (width 0.5) (layer F.Cu) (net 20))
 (segment (start 53.17099 96.46999) (end 53.221 96.52) (width 0.5) (layer F.Cu) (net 20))
 (segment (start 53.17099 67.73301) (end 53.17099 96.46999) (width 0.5) (layer F.Cu) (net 20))
 (segment (start 55.372 65.532) (end 53.17099 67.73301) (width 0.5) (layer F.Cu) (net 20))
 (segment (start 65.028 55.245) (end 66.548 55.245) (width 0.25) (layer F.Cu) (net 43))
 (segment (start 65.028 58.42) (end 66.548 58.42) (width 0.25) (layer F.Cu) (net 42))
 (via (at 72.644 58.42) (size 0.8) (drill 0.4) (layers F.Cu B.Cu) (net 6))
 (segment (start 68.123 58.42) (end 72.644 58.42) (width 0.25) (layer F.Cu) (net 6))
 (segment (start 72.644 63.5) (end 77.724 68.58) (width 0.25) (layer B.Cu) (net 6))
 (segment (start 72.644 58.42) (end 72.644 63.5) (width 0.25) (layer B.Cu) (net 6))
 (segment (start 77.724 73.279) (end 78.105 73.66) (width 0.25) (layer F.Cu) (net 6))
 (segment (start 74.76801 80.19299) (end 73.554 81.407) (width 0.25) (layer F.Cu) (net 6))
 (segment (start 73.554 81.407) (end 72.579 81.407) (width 0.25) (layer F.Cu) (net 6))
 (segment (start 79.95401 79.190254) (end 78.951274 80.19299) (width 0.25) (layer F.Cu) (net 6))
 (segment (start 79.95401 75.749746) (end 79.95401 79.190254) (width 0.25) (layer F.Cu) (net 6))
 (segment (start 78.105 73.900736) (end 79.95401 75.749746) (width 0.25) (layer F.Cu) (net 6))
 (segment (start 78.951274 80.19299) (end 74.76801 80.19299) (width 0.25) (layer F.Cu) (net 6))
 (segment (start 78.105 73.66) (end 78.105 73.900736) (width 0.25) (layer F.Cu) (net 6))
 (segment (start 77.724 73.279) (end 78.105 73.66) (width 0.25) (layer B.Cu) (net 6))
 (segment (start 77.724 68.58) (end 77.724 73.279) (width 0.25) (layer B.Cu) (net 6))
 (segment (start 65.028 61.595) (end 66.548 61.595) (width 0.25) (layer F.Cu) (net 41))
 (segment (start 74.168 80.137) (end 78.105 76.2) (width 0.25) (layer F.Cu) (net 7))
 (segment (start 72.579 80.137) (end 74.168 80.137) (width 0.25) (layer F.Cu) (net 7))
 (via (at 73.369 60.96) (size 0.8) (drill 0.4) (layers F.Cu B.Cu) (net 7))
 (segment (start 72.734 61.595) (end 73.369 60.96) (width 0.25) (layer F.Cu) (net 7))
 (segment (start 68.123 61.595) (end 72.734 61.595) (width 0.25) (layer F.Cu) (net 7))
 (segment (start 79.95401 74.35099) (end 78.105 76.2) (width 0.25) (layer B.Cu) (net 7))
 (segment (start 79.95401 67.54501) (end 79.95401 74.35099) (width 0.25) (layer B.Cu) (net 7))
 (segment (start 73.369 60.96) (end 79.95401 67.54501) (width 0.25) (layer B.Cu) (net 7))
 (segment (start 68.49 50.909998) (end 68.49 51.67) (width 0.25) (layer F.Cu) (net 44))
 (segment (start 66.856002 49.276) (end 68.49 50.909998) (width 0.25) (layer F.Cu) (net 44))
 (segment (start 65.223998 49.276) (end 66.856002 49.276) (width 0.25) (layer F.Cu) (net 44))
 (segment (start 63.59 50.909998) (end 65.223998 49.276) (width 0.25) (layer F.Cu) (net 44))
 (segment (start 63.59 51.67) (end 63.59 50.909998) (width 0.25) (layer F.Cu) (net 44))
 (via (at 65.532 50.292) (size 0.8) (drill 0.4) (layers F.Cu B.Cu) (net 36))
 (segment (start 65.79 50.55) (end 65.532 50.292) (width 0.25) (layer F.Cu) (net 36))
 (segment (start 65.79 51.67) (end 65.79 50.55) (width 0.25) (layer F.Cu) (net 36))
 (via (at 70.612 76.2) (size 0.8) (drill 0.4) (layers F.Cu B.Cu) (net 36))
 (segment (start 70.612 55.372) (end 70.612 76.2) (width 0.25) (layer B.Cu) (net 36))
 (segment (start 65.532 50.292) (end 70.612 55.372) (width 0.25) (layer B.Cu) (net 36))
 (segment (start 72.452 76.2) (end 72.579 76.327) (width 0.25) (layer F.Cu) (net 36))
 (segment (start 70.612 76.2) (end 72.452 76.2) (width 0.25) (layer F.Cu) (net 36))
 (via (at 66.575239 50.309933) (size 0.8) (drill 0.4) (layers F.Cu B.Cu) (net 37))
 (segment (start 66.29 50.595172) (end 66.575239 50.309933) (width 0.25) (layer F.Cu) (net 37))
 (segment (start 66.29 51.67) (end 66.29 50.595172) (width 0.25) (layer F.Cu) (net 37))
 (via (at 70.612 77.51699) (size 0.8) (drill 0.4) (layers F.Cu B.Cu) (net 37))
 (segment (start 71.337001 76.791989) (end 70.612 77.51699) (width 0.25) (layer B.Cu) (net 37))
 (segment (start 71.337001 55.071695) (end 71.337001 76.791989) (width 0.25) (layer B.Cu) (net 37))
 (segment (start 66.575239 50.309933) (end 71.337001 55.071695) (width 0.25) (layer B.Cu) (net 37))
 (segment (start 72.49899 77.51699) (end 72.579 77.597) (width 0.25) (layer F.Cu) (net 37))
 (segment (start 70.612 77.51699) (end 72.49899 77.51699) (width 0.25) (layer F.Cu) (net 37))
 (segment (start 75.22 52.54) (end 75.22 60.49) (width 0.25) (layer F.Cu) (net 1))
 (segment (start 75.22 60.49) (end 75.146 60.49) (width 0.25) (layer F.Cu) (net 1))
 (segment (start 72.136 63.5) (end 65.024 63.5) (width 0.25) (layer F.Cu) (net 1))
 (segment (start 75.146 60.49) (end 72.136 63.5) (width 0.25) (layer F.Cu) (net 1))
 (segment (start 55.245 81.28) (end 60.992 81.28) (width 0.25) (layer F.Cu) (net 1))
 (via (at 59.944 78.74) (size 0.8) (drill 0.4) (layers F.Cu B.Cu) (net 1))
 (segment (start 60.992 79.788) (end 59.944 78.74) (width 0.25) (layer F.Cu) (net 1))
 (segment (start 60.992 81.28) (end 60.992 79.788) (width 0.25) (layer F.Cu) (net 1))
 (segment (start 59.944 78.74) (end 65.024 73.66) (width 0.25) (layer B.Cu) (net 1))
 (via (at 65.024 65.024) (size 0.8) (drill 0.4) (layers F.Cu B.Cu) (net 1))
 (segment (start 65.024 73.66) (end 65.024 65.024) (width 0.25) (layer B.Cu) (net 1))
 (segment (start 65.024 65.024) (end 65.024 63.5) (width 0.25) (layer F.Cu) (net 1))
 (segment (start 65.909 80.137) (end 67.629 80.137) (width 0.25) (layer F.Cu) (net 30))
 (segment (start 65.024 79.252) (end 65.909 80.137) (width 0.25) (layer F.Cu) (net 30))
 (segment (start 64.511999 78.739999) (end 65.024 79.252) (width 0.25) (layer F.Cu) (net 30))
 (segment (start 63.049003 78.739999) (end 64.511999 78.739999) (width 0.25) (layer F.Cu) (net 30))
 (segment (start 62.216999 79.572003) (end 63.049003 78.739999) (width 0.25) (layer F.Cu) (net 30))
 (segment (start 62.216999 81.454999) (end 62.216999 79.572003) (width 0.25) (layer F.Cu) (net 30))
 (segment (start 62.992 82.23) (end 62.216999 81.454999) (width 0.25) (layer F.Cu) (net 30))
 (segment (start 68.005768 78.867) (end 67.629 78.867) (width 0.25) (layer F.Cu) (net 31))
 (segment (start 68.92901 80.483758) (end 68.92901 79.790242) (width 0.25) (layer F.Cu) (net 31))
 (segment (start 68.644768 80.768) (end 68.92901 80.483758) (width 0.25) (layer F.Cu) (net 31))
 (segment (start 68.92901 79.790242) (end 68.005768 78.867) (width 0.25) (layer F.Cu) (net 31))
 (segment (start 65.024 80.768) (end 68.644768 80.768) (width 0.25) (layer F.Cu) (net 31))
 (via (at 64.008 79.465) (size 0.8) (drill 0.4) (layers F.Cu B.Cu) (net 31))
 (segment (start 65.024 80.481) (end 64.008 79.465) (width 0.25) (layer F.Cu) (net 31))
 (segment (start 65.024 80.768) (end 65.024 80.481) (width 0.25) (layer F.Cu) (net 31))
 (via (at 58.928 76.708) (size 0.8) (drill 0.4) (layers F.Cu B.Cu) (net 31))
 (segment (start 58.928 78.797002) (end 58.928 76.708) (width 0.25) (layer B.Cu) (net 31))
 (segment (start 59.595998 79.465) (end 58.928 78.797002) (width 0.25) (layer B.Cu) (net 31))
 (segment (start 64.008 79.465) (end 59.595998 79.465) (width 0.25) (layer B.Cu) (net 31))
 (segment (start 60.926 76.708) (end 61.91 75.724) (width 0.25) (layer F.Cu) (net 31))
 (segment (start 58.928 76.708) (end 60.926 76.708) (width 0.25) (layer F.Cu) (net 31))
 (via (at 61.976 78.74) (size 0.8) (drill 0.4) (layers F.Cu B.Cu) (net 8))
 (segment (start 60.96 77.724) (end 61.976 78.74) (width 0.25) (layer F.Cu) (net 8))
 (segment (start 61.976 78.74) (end 78.105 78.74) (width 0.25) (layer B.Cu) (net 8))
 (segment (start 55.245 73.66) (end 60.452 73.66) (width 0.25) (layer F.Cu) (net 28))
 (segment (start 70.526999 72.709999) (end 70.526999 69.845001) (width 0.25) (layer F.Cu) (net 3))
 (segment (start 70.526999 69.845001) (end 71.452 68.92) (width 0.25) (layer F.Cu) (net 3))
 (segment (start 71.604 73.787) (end 70.526999 72.709999) (width 0.25) (layer F.Cu) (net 3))
 (segment (start 72.579 73.787) (end 71.604 73.787) (width 0.25) (layer F.Cu) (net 3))
 (segment (start 73.554 75.057) (end 72.579 75.057) (width 0.25) (layer F.Cu) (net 4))
 (segment (start 73.87901 74.73199) (end 73.554 75.057) (width 0.25) (layer F.Cu) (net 4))
 (segment (start 73.87901 71.84701) (end 73.87901 74.73199) (width 0.25) (layer F.Cu) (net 4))
 (segment (start 73.152 71.12) (end 73.87901 71.84701) (width 0.25) (layer F.Cu) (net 4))
 (segment (start 63.566 80.33) (end 65.024 81.788) (width 0.25) (layer F.Cu) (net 40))
 (segment (start 62.992 80.33) (end 63.566 80.33) (width 0.25) (layer F.Cu) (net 40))
 (segment (start 64.516 77.724) (end 65.024 78.232) (width 0.25) (layer F.Cu) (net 39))
 (segment (start 62.86 77.724) (end 64.516 77.724) (width 0.25) (layer F.Cu) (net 39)))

